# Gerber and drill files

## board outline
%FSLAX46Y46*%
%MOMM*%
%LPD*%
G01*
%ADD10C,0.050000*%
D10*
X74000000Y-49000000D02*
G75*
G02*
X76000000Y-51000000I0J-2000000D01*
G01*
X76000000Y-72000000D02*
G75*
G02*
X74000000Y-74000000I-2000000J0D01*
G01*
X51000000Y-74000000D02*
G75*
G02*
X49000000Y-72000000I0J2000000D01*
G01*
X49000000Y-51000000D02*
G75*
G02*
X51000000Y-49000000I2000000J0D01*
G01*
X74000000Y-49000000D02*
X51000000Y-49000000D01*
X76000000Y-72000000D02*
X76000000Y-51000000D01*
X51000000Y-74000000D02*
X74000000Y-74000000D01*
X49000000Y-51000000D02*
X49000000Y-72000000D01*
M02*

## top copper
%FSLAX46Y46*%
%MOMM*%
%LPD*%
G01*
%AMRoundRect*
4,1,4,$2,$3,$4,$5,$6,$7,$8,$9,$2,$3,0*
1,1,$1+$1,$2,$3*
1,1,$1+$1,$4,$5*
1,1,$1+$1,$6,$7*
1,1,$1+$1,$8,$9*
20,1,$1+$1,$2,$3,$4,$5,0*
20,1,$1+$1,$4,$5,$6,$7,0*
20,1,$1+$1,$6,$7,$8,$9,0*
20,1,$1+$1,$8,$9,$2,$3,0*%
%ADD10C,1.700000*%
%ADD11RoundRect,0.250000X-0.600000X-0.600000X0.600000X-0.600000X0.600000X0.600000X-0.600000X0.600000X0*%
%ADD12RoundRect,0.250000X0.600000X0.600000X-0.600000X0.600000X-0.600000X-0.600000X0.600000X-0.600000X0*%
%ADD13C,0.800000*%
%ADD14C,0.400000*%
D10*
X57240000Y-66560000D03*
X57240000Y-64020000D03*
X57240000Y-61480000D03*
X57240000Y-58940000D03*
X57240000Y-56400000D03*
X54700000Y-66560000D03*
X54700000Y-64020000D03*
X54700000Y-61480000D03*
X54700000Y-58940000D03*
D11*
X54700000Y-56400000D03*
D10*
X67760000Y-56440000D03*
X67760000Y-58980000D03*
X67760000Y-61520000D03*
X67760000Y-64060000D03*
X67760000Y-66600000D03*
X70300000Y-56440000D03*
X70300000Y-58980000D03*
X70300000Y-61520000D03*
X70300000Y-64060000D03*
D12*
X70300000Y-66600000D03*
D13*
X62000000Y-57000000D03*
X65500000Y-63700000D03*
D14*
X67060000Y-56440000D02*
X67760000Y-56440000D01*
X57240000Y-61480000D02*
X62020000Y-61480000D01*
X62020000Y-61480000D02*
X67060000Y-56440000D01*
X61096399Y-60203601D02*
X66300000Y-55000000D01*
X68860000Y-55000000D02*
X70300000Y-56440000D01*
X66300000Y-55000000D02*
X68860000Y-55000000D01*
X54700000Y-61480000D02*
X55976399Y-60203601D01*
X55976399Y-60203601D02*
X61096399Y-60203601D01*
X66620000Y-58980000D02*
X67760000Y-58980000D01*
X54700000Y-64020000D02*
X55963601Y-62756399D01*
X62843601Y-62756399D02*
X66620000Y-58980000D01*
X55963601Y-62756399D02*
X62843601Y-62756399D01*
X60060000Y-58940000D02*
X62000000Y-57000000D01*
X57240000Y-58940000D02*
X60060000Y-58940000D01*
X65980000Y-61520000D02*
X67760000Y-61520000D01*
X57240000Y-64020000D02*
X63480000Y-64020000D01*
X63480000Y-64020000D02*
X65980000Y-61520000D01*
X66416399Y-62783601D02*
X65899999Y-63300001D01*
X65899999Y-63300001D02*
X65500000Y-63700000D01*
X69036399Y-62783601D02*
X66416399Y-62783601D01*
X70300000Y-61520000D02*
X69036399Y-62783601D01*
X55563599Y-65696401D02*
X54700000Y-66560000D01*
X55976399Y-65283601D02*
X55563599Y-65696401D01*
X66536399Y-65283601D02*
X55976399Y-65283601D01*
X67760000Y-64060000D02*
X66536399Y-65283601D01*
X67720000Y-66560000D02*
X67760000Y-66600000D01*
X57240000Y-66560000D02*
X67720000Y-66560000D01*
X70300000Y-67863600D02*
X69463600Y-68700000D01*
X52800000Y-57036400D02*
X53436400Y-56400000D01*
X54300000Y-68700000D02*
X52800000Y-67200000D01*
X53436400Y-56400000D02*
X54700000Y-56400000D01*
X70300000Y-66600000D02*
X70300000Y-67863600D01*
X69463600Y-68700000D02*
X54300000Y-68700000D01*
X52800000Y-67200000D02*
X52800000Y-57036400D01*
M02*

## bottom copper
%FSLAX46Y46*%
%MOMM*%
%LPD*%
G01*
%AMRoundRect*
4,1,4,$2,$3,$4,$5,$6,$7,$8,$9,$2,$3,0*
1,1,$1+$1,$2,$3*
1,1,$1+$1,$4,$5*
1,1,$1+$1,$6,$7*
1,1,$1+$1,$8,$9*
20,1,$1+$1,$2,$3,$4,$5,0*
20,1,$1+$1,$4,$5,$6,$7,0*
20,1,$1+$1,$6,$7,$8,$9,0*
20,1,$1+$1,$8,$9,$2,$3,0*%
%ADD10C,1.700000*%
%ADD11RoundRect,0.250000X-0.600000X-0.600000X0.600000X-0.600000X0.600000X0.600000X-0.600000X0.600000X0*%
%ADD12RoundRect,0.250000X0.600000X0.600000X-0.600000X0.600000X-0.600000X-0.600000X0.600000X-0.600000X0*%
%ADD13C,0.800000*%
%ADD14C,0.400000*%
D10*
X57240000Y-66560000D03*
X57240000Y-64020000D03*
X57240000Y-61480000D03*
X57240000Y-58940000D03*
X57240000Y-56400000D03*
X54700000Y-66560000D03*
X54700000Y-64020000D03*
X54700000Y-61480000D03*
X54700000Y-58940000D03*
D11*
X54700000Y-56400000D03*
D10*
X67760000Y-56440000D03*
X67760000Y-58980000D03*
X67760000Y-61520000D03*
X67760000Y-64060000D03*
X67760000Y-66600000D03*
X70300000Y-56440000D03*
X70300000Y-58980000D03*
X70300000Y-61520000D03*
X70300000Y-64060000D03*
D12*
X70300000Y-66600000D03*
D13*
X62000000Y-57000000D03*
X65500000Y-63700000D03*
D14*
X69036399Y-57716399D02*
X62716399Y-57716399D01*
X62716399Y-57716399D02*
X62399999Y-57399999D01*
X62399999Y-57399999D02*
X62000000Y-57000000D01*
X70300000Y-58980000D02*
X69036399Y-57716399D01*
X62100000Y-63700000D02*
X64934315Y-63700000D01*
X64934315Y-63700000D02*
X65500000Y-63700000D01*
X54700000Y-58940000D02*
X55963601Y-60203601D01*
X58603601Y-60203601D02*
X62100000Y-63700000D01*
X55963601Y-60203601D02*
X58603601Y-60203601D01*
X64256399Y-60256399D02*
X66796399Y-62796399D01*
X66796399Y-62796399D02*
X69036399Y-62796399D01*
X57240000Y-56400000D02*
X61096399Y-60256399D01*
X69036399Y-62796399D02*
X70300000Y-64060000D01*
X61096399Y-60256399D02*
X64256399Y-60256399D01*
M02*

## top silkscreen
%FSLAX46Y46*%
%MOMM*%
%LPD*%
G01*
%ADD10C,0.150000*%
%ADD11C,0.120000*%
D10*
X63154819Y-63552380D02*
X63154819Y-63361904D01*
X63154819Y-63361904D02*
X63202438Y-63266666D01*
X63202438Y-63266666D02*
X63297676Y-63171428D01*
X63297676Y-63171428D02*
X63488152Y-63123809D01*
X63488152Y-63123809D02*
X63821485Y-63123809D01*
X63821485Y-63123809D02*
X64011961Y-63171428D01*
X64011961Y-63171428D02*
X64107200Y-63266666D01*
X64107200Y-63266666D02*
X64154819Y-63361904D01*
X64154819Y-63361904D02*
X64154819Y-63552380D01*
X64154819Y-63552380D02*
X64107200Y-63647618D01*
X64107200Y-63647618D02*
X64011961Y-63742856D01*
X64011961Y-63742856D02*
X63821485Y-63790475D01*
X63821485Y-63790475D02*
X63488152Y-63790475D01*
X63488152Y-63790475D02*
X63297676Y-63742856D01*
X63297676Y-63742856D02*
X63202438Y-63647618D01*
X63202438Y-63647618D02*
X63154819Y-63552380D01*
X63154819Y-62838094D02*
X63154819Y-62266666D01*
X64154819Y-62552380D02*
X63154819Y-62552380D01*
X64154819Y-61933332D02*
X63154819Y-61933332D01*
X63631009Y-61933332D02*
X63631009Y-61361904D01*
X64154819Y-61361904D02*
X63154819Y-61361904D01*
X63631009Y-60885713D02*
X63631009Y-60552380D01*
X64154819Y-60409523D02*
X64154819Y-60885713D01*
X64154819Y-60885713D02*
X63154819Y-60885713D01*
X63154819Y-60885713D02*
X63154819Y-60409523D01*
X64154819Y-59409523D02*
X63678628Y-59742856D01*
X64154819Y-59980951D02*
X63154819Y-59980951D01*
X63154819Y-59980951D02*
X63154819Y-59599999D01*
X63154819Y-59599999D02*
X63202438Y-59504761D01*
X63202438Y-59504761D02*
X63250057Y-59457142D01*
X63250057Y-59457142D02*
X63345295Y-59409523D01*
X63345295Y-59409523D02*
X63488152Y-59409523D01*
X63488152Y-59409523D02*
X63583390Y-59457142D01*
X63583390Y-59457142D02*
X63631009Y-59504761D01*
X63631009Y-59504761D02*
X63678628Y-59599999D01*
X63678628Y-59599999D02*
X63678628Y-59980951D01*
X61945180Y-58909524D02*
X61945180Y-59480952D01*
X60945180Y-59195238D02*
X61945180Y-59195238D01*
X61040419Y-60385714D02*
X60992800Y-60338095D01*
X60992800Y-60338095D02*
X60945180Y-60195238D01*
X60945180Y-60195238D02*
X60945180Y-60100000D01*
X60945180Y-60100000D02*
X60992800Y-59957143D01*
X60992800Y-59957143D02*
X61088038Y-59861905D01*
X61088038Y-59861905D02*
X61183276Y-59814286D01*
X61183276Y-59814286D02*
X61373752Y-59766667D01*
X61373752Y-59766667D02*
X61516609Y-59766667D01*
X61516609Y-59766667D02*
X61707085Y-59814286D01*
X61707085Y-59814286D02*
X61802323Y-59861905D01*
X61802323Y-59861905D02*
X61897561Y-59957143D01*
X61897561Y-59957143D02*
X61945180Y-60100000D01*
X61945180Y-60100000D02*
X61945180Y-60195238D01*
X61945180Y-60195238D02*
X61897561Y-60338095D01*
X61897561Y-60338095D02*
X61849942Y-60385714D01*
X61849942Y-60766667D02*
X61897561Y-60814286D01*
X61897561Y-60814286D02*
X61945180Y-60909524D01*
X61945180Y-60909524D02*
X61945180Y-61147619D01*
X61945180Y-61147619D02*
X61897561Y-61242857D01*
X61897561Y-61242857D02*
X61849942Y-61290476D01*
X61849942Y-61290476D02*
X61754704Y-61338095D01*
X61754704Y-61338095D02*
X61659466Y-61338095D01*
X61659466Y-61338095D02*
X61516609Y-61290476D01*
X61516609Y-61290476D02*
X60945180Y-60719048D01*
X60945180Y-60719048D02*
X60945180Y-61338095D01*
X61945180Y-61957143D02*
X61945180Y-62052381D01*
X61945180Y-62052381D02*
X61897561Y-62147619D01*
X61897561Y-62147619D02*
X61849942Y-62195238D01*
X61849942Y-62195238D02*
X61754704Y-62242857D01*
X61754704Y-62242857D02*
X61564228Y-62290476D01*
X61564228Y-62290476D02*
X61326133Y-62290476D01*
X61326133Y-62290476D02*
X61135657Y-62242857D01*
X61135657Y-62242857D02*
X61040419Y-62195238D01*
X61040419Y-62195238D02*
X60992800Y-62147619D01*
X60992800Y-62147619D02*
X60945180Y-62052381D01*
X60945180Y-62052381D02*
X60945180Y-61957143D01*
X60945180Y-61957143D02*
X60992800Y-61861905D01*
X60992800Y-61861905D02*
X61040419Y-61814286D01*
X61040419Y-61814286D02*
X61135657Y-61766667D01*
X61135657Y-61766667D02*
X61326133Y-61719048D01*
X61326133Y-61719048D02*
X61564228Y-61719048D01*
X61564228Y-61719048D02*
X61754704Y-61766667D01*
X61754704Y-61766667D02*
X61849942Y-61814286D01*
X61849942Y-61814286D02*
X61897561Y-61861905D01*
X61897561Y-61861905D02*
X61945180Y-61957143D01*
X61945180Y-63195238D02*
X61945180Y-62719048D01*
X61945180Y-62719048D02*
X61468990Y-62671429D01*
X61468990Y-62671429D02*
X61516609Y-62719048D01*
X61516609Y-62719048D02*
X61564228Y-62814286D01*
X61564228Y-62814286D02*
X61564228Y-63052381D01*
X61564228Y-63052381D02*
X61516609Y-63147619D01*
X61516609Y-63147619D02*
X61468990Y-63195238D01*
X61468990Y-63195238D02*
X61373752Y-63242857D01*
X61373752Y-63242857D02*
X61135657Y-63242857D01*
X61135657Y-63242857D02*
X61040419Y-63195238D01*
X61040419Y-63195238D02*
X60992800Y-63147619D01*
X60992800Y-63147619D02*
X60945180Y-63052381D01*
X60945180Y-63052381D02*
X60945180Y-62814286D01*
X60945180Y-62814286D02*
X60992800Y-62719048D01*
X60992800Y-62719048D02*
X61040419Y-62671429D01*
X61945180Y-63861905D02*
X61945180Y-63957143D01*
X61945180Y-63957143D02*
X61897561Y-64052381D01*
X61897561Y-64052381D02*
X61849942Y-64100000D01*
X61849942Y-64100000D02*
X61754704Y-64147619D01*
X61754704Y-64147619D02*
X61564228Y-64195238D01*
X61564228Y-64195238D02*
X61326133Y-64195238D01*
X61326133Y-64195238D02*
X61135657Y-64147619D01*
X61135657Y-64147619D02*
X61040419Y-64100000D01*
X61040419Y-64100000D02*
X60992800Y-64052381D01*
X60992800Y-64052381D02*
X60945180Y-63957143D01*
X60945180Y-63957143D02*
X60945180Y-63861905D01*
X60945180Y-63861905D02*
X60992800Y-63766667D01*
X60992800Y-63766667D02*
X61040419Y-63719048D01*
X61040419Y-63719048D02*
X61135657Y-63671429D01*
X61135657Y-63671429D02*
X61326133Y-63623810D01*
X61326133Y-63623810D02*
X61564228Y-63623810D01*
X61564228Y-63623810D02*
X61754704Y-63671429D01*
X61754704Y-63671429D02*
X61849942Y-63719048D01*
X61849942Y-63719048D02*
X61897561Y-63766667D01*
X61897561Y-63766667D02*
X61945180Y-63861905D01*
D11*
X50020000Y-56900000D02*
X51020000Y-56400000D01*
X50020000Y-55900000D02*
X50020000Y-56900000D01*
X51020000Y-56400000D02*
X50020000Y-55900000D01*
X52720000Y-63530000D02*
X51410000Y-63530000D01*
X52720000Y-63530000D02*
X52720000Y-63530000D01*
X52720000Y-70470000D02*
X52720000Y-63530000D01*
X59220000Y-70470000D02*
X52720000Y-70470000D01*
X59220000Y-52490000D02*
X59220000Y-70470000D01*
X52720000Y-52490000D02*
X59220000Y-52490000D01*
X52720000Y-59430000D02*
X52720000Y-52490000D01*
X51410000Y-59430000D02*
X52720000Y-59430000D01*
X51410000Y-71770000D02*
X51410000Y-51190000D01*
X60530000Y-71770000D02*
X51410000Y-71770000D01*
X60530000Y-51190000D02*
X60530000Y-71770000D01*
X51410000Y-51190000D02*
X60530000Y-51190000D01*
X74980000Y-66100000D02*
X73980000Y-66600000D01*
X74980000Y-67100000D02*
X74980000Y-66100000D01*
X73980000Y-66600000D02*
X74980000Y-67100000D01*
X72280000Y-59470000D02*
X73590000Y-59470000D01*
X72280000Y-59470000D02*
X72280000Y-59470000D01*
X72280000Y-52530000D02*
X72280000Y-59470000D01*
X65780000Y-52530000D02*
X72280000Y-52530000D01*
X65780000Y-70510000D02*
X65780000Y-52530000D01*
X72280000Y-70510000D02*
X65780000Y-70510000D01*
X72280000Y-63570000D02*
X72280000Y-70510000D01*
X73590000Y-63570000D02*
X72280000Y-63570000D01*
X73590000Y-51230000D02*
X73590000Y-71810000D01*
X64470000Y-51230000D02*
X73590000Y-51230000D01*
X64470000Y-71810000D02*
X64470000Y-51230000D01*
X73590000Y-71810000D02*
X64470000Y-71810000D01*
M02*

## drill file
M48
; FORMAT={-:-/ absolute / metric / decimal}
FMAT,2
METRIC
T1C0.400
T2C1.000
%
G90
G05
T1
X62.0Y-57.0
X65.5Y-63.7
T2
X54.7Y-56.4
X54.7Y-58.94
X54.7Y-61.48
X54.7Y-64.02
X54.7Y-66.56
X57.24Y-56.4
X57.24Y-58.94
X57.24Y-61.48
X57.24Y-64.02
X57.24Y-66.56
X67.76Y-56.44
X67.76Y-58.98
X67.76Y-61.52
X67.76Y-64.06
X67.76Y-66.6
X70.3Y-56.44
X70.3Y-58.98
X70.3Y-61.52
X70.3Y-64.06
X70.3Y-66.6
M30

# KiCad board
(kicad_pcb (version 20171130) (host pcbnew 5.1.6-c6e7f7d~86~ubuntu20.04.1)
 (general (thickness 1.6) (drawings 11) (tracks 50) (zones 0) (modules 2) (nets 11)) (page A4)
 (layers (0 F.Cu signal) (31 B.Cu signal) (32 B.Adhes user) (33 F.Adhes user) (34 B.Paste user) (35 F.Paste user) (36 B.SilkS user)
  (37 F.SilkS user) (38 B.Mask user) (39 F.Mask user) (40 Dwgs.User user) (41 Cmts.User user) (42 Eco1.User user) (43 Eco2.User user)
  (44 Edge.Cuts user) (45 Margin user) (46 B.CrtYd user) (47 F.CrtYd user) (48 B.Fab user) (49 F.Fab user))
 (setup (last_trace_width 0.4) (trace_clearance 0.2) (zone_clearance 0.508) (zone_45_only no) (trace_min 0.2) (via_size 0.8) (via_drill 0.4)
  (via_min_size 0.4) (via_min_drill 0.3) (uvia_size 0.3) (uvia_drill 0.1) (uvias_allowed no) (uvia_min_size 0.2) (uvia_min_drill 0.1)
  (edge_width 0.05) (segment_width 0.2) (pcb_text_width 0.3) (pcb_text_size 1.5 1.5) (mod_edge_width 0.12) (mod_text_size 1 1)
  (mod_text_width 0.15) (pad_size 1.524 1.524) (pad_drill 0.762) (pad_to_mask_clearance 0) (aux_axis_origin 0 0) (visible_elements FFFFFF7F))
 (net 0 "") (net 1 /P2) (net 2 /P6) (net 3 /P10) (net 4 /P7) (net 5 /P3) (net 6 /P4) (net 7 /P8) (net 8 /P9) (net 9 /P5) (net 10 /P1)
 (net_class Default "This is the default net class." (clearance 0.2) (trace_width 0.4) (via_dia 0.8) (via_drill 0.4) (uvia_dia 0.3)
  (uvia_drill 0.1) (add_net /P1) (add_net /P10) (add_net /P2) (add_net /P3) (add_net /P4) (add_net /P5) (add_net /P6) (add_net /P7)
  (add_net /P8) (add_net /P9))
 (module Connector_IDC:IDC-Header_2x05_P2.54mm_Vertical (layer F.Cu) (at 54.7 56.4)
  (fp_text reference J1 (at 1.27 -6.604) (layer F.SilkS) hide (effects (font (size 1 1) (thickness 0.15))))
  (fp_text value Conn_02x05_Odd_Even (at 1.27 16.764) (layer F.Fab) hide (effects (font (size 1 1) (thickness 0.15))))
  (fp_line (start -4.68 0.5) (end -3.68 0) (layer F.SilkS) (width 0.12))
  (fp_line (start -4.68 -0.5) (end -4.68 0.5) (layer F.SilkS) (width 0.12))
  (fp_line (start -3.68 0) (end -4.68 -0.5) (layer F.SilkS) (width 0.12))
  (fp_line (start -1.98 7.13) (end -3.29 7.13) (layer F.SilkS) (width 0.12))
  (fp_line (start -1.98 7.13) (end -1.98 7.13) (layer F.SilkS) (width 0.12))
  (fp_line (start -1.98 14.07) (end -1.98 7.13) (layer F.SilkS) (width 0.12))
  (fp_line (start 4.52 14.07) (end -1.98 14.07) (layer F.SilkS) (width 0.12))
  (fp_line (start 4.52 -3.91) (end 4.52 14.07) (layer F.SilkS) (width 0.12))
  (fp_line (start -1.98 -3.91) (end 4.52 -3.91) (layer F.SilkS) (width 0.12))
  (fp_line (start -1.98 3.03) (end -1.98 -3.91) (layer F.SilkS) (width 0.12))
  (fp_line (start -3.29 3.03) (end -1.98 3.03) (layer F.SilkS) (width 0.12))
  (fp_line (start -3.29 15.37) (end -3.29 -5.21) (layer F.SilkS) (width 0.12))
  (fp_line (start 5.83 15.37) (end -3.29 15.37) (layer F.SilkS) (width 0.12))
  (fp_line (start 5.83 -5.21) (end 5.83 15.37) (layer F.SilkS) (width 0.12))
  (fp_line (start -3.29 -5.21) (end 5.83 -5.21) (layer F.SilkS) (width 0.12))
  (pad 10 thru_hole circle (at 2.54 10.16) (size 1.7 1.7) (drill 1) (layers *.Cu *.Mask) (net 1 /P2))
  (pad 8 thru_hole circle (at 2.54 7.62) (size 1.7 1.7) (drill 1) (layers *.Cu *.Mask) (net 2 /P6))
  (pad 6 thru_hole circle (at 2.54 5.08) (size 1.7 1.7) (drill 1) (layers *.Cu *.Mask) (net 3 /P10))
  (pad 4 thru_hole circle (at 2.54 2.54) (size 1.7 1.7) (drill 1) (layers *.Cu *.Mask) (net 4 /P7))
  (pad 2 thru_hole circle (at 2.54 0) (size 1.7 1.7) (drill 1) (layers *.Cu *.Mask) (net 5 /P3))
  (pad 9 thru_hole circle (at 0 10.16) (size 1.7 1.7) (drill 1) (layers *.Cu *.Mask) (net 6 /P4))
  (pad 7 thru_hole circle (at 0 7.62) (size 1.7 1.7) (drill 1) (layers *.Cu *.Mask) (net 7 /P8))
  (pad 5 thru_hole circle (at 0 5.08) (size 1.7 1.7) (drill 1) (layers *.Cu *.Mask) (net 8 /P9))
  (pad 3 thru_hole circle (at 0 2.54) (size 1.7 1.7) (drill 1) (layers *.Cu *.Mask) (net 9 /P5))
  (pad 1 thru_hole roundrect (at 0 0) (size 1.7 1.7) (drill 1) (layers *.Cu *.Mask) (roundrect_rratio 0.147059) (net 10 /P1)))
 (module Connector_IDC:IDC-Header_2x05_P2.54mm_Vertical (layer F.Cu) (at 70.3 66.6 180)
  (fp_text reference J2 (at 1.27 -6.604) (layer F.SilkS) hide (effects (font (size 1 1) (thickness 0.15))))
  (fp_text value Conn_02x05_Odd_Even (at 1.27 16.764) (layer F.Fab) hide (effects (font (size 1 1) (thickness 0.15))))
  (fp_line (start -4.68 0.5) (end -3.68 0) (layer F.SilkS) (width 0.12))
  (fp_line (start -4.68 -0.5) (end -4.68 0.5) (layer F.SilkS) (width 0.12))
  (fp_line (start -3.68 0) (end -4.68 -0.5) (layer F.SilkS) (width 0.12))
  (fp_line (start -1.98 7.13) (end -3.29 7.13) (layer F.SilkS) (width 0.12))
  (fp_line (start -1.98 7.13) (end -1.98 7.13) (layer F.SilkS) (width 0.12))
  (fp_line (start -1.98 14.07) (end -1.98 7.13) (layer F.SilkS) (width 0.12))
  (fp_line (start 4.52 14.07) (end -1.98 14.07) (layer F.SilkS) (width 0.12))
  (fp_line (start 4.52 -3.91) (end 4.52 14.07) (layer F.SilkS) (width 0.12))
  (fp_line (start -1.98 -3.91) (end 4.52 -3.91) (layer F.SilkS) (width 0.12))
  (fp_line (start -1.98 3.03) (end -1.98 -3.91) (layer F.SilkS) (width 0.12))
  (fp_line (start -3.29 3.03) (end -1.98 3.03) (layer F.SilkS) (width 0.12))
  (fp_line (start -3.29 15.37) (end -3.29 -5.21) (layer F.SilkS) (width 0.12))
  (fp_line (start 5.83 15.37) (end -3.29 15.37) (layer F.SilkS) (width 0.12))
  (fp_line (start 5.83 -5.21) (end 5.83 15.37) (layer F.SilkS) (width 0.12))
  (fp_line (start -3.29 -5.21) (end 5.83 -5.21) (layer F.SilkS) (width 0.12))
  (pad 10 thru_hole circle (at 2.54 10.16 180) (size 1.7 1.7) (drill 1) (layers *.Cu *.Mask) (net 3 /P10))
  (pad 8 thru_hole circle (at 2.54 7.62 180) (size 1.7 1.7) (drill 1) (layers *.Cu *.Mask) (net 7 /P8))
  (pad 6 thru_hole circle (at 2.54 5.08 180) (size 1.7 1.7) (drill 1) (layers *.Cu *.Mask) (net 2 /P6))
  (pad 4 thru_hole circle (at 2.54 2.54 180) (size 1.7 1.7) (drill 1) (layers *.Cu *.Mask) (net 6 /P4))
  (pad 2 thru_hole circle (at 2.54 0 180) (size 1.7 1.7) (drill 1) (layers *.Cu *.Mask) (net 1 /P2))
  (pad 9 thru_hole circle (at 0 10.16 180) (size 1.7 1.7) (drill 1) (layers *.Cu *.Mask) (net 8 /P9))
  (pad 7 thru_hole circle (at 0 7.62 180) (size 1.7 1.7) (drill 1) (layers *.Cu *.Mask) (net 4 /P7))
  (pad 5 thru_hole circle (at 0 5.08 180) (size 1.7 1.7) (drill 1) (layers *.Cu *.Mask) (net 9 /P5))
  (pad 3 thru_hole circle (at 0 2.54 180) (size 1.7 1.7) (drill 1) (layers *.Cu *.Mask) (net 5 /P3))
  (pad 1 thru_hole roundrect (at 0 0 180) (size 1.7 1.7) (drill 1) (layers *.Cu *.Mask) (roundrect_rratio 0.147059) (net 10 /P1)))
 (gr_arc (start 74 51) (end 76 51) (angle -90) (layer Edge.Cuts) (width 0.05))
 (gr_arc (start 74 72) (end 74 74) (angle -90) (layer Edge.Cuts) (width 0.05))
 (gr_arc (start 51 72) (end 49 72) (angle -90) (layer Edge.Cuts) (width 0.05))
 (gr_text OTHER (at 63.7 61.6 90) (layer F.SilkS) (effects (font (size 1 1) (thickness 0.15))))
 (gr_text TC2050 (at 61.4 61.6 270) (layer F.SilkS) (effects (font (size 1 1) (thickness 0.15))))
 (gr_arc (start 51 51) (end 51 49) (angle -90) (layer Edge.Cuts) (width 0.05))
 (gr_line (start 74 49) (end 51 49) (layer Edge.Cuts) (width 0.05))
 (gr_line (start 76 72) (end 76 51) (layer Edge.Cuts) (width 0.05))
 (gr_line (start 51 74) (end 74 74) (layer Edge.Cuts) (width 0.05))
 (gr_line (start 49 51) (end 49 72) (layer Edge.Cuts) (width 0.05))
 (segment (start 67.06 56.44) (end 67.76 56.44) (width 0.4) (layer F.Cu) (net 3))
 (segment (start 57.24 61.48) (end 62.02 61.48) (width 0.4) (layer F.Cu) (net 3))
 (segment (start 62.02 61.48) (end 67.06 56.44) (width 0.4) (layer F.Cu) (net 3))
 (segment (start 61.096399 60.203601) (end 66.3 55) (width 0.4) (layer F.Cu) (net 8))
 (segment (start 68.86 55) (end 70.3 56.44) (width 0.4) (layer F.Cu) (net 8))
 (segment (start 66.3 55) (end 68.86 55) (width 0.4) (layer F.Cu) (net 8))
 (segment (start 54.7 61.48) (end 55.976399 60.203601) (width 0.4) (layer F.Cu) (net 8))
 (segment (start 55.976399 60.203601) (end 61.096399 60.203601) (width 0.4) (layer F.Cu) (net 8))
 (segment (start 66.62 58.98) (end 67.76 58.98) (width 0.4) (layer F.Cu) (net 7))
 (segment (start 54.7 64.02) (end 55.963601 62.756399) (width 0.4) (layer F.Cu) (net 7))
 (segment (start 62.843601 62.756399) (end 66.62 58.98) (width 0.4) (layer F.Cu) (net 7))
 (segment (start 55.963601 62.756399) (end 62.843601 62.756399) (width 0.4) (layer F.Cu) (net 7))
 (segment (start 69.036399 57.716399) (end 62.716399 57.716399) (width 0.4) (layer B.Cu) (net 4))
 (segment (start 62.716399 57.716399) (end 62.399999 57.399999) (width 0.4) (layer B.Cu) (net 4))
 (segment (start 60.06 58.94) (end 62 57) (width 0.4) (layer F.Cu) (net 4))
 (via (at 62 57) (size 0.8) (drill 0.4) (layers F.Cu B.Cu) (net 4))
 (segment (start 62.399999 57.399999) (end 62 57) (width 0.4) (layer B.Cu) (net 4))
 (segment (start 70.3 58.98) (end 69.036399 57.716399) (width 0.4) (layer B.Cu) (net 4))
 (segment (start 57.24 58.94) (end 60.06 58.94) (width 0.4) (layer F.Cu) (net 4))
 (segment (start 65.98 61.52) (end 67.76 61.52) (width 0.4) (layer F.Cu) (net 2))
 (segment (start 57.24 64.02) (end 63.48 64.02) (width 0.4) (layer F.Cu) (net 2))
 (segment (start 63.48 64.02) (end 65.98 61.52) (width 0.4) (layer F.Cu) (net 2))
 (segment (start 62.1 63.7) (end 64.934315 63.7) (width 0.4) (layer B.Cu) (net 9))
 (segment (start 66.416399 62.783601) (end 65.899999 63.300001) (width 0.4) (layer F.Cu) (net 9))
 (segment (start 64.934315 63.7) (end 65.5 63.7) (width 0.4) (layer B.Cu) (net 9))
 (segment (start 54.7 58.94) (end 55.963601 60.203601) (width 0.4) (layer B.Cu) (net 9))
 (segment (start 58.603601 60.203601) (end 62.1 63.7) (width 0.4) (layer B.Cu) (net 9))
 (segment (start 65.899999 63.300001) (end 65.5 63.7) (width 0.4) (layer F.Cu) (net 9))
 (segment (start 69.036399 62.783601) (end 66.416399 62.783601) (width 0.4) (layer F.Cu) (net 9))
 (via (at 65.5 63.7) (size 0.8) (drill 0.4) (layers F.Cu B.Cu) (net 9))
 (segment (start 55.963601 60.203601) (end 58.603601 60.203601) (width 0.4) (layer B.Cu) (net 9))
 (segment (start 70.3 61.52) (end 69.036399 62.783601) (width 0.4) (layer F.Cu) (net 9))
 (segment (start 55.563599 65.696401) (end 54.7 66.56) (width 0.4) (layer F.Cu) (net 6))
 (segment (start 55.976399 65.283601) (end 55.563599 65.696401) (width 0.4) (layer F.Cu) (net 6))
 (segment (start 66.536399 65.283601) (end 55.976399 65.283601) (width 0.4) (layer F.Cu) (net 6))
 (segment (start 67.76 64.06) (end 66.536399 65.283601) (width 0.4) (layer F.Cu) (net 6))
 (segment (start 64.256399 60.256399) (end 66.796399 62.796399) (width 0.4) (layer B.Cu) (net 5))
 (segment (start 66.796399 62.796399) (end 69.036399 62.796399) (width 0.4) (layer B.Cu) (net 5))
 (segment (start 57.24 56.4) (end 61.096399 60.256399) (width 0.4) (layer B.Cu) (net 5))
 (segment (start 69.036399 62.796399) (end 70.3 64.06) (width 0.4) (layer B.Cu) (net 5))
 (segment (start 61.096399 60.256399) (end 64.256399 60.256399) (width 0.4) (layer B.Cu) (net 5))
 (segment (start 67.72 66.56) (end 67.76 66.6) (width 0.4) (layer F.Cu) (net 1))
 (segment (start 57.24 66.56) (end 67.72 66.56) (width 0.4) (layer F.Cu) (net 1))
 (segment (start 70.3 67.8636) (end 69.4636 68.7) (width 0.4) (layer F.Cu) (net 10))
 (segment (start 52.8 57.0364) (end 53.4364 56.4) (width 0.4) (layer F.Cu) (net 10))
 (segment (start 54.3 68.7) (end 52.8 67.2) (width 0.4) (layer F.Cu) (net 10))
 (segment (start 53.4364 56.4) (end 54.7 56.4) (width 0.4) (layer F.Cu) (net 10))
 (segment (start 70.3 66.6) (end 70.3 67.8636) (width 0.4) (layer F.Cu) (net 10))
 (segment (start 69.4636 68.7) (end 54.3 68.7) (width 0.4) (layer F.Cu) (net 10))
 (segment (start 52.8 67.2) (end 52.8 57.0364) (width 0.4) (layer F.Cu) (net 10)))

